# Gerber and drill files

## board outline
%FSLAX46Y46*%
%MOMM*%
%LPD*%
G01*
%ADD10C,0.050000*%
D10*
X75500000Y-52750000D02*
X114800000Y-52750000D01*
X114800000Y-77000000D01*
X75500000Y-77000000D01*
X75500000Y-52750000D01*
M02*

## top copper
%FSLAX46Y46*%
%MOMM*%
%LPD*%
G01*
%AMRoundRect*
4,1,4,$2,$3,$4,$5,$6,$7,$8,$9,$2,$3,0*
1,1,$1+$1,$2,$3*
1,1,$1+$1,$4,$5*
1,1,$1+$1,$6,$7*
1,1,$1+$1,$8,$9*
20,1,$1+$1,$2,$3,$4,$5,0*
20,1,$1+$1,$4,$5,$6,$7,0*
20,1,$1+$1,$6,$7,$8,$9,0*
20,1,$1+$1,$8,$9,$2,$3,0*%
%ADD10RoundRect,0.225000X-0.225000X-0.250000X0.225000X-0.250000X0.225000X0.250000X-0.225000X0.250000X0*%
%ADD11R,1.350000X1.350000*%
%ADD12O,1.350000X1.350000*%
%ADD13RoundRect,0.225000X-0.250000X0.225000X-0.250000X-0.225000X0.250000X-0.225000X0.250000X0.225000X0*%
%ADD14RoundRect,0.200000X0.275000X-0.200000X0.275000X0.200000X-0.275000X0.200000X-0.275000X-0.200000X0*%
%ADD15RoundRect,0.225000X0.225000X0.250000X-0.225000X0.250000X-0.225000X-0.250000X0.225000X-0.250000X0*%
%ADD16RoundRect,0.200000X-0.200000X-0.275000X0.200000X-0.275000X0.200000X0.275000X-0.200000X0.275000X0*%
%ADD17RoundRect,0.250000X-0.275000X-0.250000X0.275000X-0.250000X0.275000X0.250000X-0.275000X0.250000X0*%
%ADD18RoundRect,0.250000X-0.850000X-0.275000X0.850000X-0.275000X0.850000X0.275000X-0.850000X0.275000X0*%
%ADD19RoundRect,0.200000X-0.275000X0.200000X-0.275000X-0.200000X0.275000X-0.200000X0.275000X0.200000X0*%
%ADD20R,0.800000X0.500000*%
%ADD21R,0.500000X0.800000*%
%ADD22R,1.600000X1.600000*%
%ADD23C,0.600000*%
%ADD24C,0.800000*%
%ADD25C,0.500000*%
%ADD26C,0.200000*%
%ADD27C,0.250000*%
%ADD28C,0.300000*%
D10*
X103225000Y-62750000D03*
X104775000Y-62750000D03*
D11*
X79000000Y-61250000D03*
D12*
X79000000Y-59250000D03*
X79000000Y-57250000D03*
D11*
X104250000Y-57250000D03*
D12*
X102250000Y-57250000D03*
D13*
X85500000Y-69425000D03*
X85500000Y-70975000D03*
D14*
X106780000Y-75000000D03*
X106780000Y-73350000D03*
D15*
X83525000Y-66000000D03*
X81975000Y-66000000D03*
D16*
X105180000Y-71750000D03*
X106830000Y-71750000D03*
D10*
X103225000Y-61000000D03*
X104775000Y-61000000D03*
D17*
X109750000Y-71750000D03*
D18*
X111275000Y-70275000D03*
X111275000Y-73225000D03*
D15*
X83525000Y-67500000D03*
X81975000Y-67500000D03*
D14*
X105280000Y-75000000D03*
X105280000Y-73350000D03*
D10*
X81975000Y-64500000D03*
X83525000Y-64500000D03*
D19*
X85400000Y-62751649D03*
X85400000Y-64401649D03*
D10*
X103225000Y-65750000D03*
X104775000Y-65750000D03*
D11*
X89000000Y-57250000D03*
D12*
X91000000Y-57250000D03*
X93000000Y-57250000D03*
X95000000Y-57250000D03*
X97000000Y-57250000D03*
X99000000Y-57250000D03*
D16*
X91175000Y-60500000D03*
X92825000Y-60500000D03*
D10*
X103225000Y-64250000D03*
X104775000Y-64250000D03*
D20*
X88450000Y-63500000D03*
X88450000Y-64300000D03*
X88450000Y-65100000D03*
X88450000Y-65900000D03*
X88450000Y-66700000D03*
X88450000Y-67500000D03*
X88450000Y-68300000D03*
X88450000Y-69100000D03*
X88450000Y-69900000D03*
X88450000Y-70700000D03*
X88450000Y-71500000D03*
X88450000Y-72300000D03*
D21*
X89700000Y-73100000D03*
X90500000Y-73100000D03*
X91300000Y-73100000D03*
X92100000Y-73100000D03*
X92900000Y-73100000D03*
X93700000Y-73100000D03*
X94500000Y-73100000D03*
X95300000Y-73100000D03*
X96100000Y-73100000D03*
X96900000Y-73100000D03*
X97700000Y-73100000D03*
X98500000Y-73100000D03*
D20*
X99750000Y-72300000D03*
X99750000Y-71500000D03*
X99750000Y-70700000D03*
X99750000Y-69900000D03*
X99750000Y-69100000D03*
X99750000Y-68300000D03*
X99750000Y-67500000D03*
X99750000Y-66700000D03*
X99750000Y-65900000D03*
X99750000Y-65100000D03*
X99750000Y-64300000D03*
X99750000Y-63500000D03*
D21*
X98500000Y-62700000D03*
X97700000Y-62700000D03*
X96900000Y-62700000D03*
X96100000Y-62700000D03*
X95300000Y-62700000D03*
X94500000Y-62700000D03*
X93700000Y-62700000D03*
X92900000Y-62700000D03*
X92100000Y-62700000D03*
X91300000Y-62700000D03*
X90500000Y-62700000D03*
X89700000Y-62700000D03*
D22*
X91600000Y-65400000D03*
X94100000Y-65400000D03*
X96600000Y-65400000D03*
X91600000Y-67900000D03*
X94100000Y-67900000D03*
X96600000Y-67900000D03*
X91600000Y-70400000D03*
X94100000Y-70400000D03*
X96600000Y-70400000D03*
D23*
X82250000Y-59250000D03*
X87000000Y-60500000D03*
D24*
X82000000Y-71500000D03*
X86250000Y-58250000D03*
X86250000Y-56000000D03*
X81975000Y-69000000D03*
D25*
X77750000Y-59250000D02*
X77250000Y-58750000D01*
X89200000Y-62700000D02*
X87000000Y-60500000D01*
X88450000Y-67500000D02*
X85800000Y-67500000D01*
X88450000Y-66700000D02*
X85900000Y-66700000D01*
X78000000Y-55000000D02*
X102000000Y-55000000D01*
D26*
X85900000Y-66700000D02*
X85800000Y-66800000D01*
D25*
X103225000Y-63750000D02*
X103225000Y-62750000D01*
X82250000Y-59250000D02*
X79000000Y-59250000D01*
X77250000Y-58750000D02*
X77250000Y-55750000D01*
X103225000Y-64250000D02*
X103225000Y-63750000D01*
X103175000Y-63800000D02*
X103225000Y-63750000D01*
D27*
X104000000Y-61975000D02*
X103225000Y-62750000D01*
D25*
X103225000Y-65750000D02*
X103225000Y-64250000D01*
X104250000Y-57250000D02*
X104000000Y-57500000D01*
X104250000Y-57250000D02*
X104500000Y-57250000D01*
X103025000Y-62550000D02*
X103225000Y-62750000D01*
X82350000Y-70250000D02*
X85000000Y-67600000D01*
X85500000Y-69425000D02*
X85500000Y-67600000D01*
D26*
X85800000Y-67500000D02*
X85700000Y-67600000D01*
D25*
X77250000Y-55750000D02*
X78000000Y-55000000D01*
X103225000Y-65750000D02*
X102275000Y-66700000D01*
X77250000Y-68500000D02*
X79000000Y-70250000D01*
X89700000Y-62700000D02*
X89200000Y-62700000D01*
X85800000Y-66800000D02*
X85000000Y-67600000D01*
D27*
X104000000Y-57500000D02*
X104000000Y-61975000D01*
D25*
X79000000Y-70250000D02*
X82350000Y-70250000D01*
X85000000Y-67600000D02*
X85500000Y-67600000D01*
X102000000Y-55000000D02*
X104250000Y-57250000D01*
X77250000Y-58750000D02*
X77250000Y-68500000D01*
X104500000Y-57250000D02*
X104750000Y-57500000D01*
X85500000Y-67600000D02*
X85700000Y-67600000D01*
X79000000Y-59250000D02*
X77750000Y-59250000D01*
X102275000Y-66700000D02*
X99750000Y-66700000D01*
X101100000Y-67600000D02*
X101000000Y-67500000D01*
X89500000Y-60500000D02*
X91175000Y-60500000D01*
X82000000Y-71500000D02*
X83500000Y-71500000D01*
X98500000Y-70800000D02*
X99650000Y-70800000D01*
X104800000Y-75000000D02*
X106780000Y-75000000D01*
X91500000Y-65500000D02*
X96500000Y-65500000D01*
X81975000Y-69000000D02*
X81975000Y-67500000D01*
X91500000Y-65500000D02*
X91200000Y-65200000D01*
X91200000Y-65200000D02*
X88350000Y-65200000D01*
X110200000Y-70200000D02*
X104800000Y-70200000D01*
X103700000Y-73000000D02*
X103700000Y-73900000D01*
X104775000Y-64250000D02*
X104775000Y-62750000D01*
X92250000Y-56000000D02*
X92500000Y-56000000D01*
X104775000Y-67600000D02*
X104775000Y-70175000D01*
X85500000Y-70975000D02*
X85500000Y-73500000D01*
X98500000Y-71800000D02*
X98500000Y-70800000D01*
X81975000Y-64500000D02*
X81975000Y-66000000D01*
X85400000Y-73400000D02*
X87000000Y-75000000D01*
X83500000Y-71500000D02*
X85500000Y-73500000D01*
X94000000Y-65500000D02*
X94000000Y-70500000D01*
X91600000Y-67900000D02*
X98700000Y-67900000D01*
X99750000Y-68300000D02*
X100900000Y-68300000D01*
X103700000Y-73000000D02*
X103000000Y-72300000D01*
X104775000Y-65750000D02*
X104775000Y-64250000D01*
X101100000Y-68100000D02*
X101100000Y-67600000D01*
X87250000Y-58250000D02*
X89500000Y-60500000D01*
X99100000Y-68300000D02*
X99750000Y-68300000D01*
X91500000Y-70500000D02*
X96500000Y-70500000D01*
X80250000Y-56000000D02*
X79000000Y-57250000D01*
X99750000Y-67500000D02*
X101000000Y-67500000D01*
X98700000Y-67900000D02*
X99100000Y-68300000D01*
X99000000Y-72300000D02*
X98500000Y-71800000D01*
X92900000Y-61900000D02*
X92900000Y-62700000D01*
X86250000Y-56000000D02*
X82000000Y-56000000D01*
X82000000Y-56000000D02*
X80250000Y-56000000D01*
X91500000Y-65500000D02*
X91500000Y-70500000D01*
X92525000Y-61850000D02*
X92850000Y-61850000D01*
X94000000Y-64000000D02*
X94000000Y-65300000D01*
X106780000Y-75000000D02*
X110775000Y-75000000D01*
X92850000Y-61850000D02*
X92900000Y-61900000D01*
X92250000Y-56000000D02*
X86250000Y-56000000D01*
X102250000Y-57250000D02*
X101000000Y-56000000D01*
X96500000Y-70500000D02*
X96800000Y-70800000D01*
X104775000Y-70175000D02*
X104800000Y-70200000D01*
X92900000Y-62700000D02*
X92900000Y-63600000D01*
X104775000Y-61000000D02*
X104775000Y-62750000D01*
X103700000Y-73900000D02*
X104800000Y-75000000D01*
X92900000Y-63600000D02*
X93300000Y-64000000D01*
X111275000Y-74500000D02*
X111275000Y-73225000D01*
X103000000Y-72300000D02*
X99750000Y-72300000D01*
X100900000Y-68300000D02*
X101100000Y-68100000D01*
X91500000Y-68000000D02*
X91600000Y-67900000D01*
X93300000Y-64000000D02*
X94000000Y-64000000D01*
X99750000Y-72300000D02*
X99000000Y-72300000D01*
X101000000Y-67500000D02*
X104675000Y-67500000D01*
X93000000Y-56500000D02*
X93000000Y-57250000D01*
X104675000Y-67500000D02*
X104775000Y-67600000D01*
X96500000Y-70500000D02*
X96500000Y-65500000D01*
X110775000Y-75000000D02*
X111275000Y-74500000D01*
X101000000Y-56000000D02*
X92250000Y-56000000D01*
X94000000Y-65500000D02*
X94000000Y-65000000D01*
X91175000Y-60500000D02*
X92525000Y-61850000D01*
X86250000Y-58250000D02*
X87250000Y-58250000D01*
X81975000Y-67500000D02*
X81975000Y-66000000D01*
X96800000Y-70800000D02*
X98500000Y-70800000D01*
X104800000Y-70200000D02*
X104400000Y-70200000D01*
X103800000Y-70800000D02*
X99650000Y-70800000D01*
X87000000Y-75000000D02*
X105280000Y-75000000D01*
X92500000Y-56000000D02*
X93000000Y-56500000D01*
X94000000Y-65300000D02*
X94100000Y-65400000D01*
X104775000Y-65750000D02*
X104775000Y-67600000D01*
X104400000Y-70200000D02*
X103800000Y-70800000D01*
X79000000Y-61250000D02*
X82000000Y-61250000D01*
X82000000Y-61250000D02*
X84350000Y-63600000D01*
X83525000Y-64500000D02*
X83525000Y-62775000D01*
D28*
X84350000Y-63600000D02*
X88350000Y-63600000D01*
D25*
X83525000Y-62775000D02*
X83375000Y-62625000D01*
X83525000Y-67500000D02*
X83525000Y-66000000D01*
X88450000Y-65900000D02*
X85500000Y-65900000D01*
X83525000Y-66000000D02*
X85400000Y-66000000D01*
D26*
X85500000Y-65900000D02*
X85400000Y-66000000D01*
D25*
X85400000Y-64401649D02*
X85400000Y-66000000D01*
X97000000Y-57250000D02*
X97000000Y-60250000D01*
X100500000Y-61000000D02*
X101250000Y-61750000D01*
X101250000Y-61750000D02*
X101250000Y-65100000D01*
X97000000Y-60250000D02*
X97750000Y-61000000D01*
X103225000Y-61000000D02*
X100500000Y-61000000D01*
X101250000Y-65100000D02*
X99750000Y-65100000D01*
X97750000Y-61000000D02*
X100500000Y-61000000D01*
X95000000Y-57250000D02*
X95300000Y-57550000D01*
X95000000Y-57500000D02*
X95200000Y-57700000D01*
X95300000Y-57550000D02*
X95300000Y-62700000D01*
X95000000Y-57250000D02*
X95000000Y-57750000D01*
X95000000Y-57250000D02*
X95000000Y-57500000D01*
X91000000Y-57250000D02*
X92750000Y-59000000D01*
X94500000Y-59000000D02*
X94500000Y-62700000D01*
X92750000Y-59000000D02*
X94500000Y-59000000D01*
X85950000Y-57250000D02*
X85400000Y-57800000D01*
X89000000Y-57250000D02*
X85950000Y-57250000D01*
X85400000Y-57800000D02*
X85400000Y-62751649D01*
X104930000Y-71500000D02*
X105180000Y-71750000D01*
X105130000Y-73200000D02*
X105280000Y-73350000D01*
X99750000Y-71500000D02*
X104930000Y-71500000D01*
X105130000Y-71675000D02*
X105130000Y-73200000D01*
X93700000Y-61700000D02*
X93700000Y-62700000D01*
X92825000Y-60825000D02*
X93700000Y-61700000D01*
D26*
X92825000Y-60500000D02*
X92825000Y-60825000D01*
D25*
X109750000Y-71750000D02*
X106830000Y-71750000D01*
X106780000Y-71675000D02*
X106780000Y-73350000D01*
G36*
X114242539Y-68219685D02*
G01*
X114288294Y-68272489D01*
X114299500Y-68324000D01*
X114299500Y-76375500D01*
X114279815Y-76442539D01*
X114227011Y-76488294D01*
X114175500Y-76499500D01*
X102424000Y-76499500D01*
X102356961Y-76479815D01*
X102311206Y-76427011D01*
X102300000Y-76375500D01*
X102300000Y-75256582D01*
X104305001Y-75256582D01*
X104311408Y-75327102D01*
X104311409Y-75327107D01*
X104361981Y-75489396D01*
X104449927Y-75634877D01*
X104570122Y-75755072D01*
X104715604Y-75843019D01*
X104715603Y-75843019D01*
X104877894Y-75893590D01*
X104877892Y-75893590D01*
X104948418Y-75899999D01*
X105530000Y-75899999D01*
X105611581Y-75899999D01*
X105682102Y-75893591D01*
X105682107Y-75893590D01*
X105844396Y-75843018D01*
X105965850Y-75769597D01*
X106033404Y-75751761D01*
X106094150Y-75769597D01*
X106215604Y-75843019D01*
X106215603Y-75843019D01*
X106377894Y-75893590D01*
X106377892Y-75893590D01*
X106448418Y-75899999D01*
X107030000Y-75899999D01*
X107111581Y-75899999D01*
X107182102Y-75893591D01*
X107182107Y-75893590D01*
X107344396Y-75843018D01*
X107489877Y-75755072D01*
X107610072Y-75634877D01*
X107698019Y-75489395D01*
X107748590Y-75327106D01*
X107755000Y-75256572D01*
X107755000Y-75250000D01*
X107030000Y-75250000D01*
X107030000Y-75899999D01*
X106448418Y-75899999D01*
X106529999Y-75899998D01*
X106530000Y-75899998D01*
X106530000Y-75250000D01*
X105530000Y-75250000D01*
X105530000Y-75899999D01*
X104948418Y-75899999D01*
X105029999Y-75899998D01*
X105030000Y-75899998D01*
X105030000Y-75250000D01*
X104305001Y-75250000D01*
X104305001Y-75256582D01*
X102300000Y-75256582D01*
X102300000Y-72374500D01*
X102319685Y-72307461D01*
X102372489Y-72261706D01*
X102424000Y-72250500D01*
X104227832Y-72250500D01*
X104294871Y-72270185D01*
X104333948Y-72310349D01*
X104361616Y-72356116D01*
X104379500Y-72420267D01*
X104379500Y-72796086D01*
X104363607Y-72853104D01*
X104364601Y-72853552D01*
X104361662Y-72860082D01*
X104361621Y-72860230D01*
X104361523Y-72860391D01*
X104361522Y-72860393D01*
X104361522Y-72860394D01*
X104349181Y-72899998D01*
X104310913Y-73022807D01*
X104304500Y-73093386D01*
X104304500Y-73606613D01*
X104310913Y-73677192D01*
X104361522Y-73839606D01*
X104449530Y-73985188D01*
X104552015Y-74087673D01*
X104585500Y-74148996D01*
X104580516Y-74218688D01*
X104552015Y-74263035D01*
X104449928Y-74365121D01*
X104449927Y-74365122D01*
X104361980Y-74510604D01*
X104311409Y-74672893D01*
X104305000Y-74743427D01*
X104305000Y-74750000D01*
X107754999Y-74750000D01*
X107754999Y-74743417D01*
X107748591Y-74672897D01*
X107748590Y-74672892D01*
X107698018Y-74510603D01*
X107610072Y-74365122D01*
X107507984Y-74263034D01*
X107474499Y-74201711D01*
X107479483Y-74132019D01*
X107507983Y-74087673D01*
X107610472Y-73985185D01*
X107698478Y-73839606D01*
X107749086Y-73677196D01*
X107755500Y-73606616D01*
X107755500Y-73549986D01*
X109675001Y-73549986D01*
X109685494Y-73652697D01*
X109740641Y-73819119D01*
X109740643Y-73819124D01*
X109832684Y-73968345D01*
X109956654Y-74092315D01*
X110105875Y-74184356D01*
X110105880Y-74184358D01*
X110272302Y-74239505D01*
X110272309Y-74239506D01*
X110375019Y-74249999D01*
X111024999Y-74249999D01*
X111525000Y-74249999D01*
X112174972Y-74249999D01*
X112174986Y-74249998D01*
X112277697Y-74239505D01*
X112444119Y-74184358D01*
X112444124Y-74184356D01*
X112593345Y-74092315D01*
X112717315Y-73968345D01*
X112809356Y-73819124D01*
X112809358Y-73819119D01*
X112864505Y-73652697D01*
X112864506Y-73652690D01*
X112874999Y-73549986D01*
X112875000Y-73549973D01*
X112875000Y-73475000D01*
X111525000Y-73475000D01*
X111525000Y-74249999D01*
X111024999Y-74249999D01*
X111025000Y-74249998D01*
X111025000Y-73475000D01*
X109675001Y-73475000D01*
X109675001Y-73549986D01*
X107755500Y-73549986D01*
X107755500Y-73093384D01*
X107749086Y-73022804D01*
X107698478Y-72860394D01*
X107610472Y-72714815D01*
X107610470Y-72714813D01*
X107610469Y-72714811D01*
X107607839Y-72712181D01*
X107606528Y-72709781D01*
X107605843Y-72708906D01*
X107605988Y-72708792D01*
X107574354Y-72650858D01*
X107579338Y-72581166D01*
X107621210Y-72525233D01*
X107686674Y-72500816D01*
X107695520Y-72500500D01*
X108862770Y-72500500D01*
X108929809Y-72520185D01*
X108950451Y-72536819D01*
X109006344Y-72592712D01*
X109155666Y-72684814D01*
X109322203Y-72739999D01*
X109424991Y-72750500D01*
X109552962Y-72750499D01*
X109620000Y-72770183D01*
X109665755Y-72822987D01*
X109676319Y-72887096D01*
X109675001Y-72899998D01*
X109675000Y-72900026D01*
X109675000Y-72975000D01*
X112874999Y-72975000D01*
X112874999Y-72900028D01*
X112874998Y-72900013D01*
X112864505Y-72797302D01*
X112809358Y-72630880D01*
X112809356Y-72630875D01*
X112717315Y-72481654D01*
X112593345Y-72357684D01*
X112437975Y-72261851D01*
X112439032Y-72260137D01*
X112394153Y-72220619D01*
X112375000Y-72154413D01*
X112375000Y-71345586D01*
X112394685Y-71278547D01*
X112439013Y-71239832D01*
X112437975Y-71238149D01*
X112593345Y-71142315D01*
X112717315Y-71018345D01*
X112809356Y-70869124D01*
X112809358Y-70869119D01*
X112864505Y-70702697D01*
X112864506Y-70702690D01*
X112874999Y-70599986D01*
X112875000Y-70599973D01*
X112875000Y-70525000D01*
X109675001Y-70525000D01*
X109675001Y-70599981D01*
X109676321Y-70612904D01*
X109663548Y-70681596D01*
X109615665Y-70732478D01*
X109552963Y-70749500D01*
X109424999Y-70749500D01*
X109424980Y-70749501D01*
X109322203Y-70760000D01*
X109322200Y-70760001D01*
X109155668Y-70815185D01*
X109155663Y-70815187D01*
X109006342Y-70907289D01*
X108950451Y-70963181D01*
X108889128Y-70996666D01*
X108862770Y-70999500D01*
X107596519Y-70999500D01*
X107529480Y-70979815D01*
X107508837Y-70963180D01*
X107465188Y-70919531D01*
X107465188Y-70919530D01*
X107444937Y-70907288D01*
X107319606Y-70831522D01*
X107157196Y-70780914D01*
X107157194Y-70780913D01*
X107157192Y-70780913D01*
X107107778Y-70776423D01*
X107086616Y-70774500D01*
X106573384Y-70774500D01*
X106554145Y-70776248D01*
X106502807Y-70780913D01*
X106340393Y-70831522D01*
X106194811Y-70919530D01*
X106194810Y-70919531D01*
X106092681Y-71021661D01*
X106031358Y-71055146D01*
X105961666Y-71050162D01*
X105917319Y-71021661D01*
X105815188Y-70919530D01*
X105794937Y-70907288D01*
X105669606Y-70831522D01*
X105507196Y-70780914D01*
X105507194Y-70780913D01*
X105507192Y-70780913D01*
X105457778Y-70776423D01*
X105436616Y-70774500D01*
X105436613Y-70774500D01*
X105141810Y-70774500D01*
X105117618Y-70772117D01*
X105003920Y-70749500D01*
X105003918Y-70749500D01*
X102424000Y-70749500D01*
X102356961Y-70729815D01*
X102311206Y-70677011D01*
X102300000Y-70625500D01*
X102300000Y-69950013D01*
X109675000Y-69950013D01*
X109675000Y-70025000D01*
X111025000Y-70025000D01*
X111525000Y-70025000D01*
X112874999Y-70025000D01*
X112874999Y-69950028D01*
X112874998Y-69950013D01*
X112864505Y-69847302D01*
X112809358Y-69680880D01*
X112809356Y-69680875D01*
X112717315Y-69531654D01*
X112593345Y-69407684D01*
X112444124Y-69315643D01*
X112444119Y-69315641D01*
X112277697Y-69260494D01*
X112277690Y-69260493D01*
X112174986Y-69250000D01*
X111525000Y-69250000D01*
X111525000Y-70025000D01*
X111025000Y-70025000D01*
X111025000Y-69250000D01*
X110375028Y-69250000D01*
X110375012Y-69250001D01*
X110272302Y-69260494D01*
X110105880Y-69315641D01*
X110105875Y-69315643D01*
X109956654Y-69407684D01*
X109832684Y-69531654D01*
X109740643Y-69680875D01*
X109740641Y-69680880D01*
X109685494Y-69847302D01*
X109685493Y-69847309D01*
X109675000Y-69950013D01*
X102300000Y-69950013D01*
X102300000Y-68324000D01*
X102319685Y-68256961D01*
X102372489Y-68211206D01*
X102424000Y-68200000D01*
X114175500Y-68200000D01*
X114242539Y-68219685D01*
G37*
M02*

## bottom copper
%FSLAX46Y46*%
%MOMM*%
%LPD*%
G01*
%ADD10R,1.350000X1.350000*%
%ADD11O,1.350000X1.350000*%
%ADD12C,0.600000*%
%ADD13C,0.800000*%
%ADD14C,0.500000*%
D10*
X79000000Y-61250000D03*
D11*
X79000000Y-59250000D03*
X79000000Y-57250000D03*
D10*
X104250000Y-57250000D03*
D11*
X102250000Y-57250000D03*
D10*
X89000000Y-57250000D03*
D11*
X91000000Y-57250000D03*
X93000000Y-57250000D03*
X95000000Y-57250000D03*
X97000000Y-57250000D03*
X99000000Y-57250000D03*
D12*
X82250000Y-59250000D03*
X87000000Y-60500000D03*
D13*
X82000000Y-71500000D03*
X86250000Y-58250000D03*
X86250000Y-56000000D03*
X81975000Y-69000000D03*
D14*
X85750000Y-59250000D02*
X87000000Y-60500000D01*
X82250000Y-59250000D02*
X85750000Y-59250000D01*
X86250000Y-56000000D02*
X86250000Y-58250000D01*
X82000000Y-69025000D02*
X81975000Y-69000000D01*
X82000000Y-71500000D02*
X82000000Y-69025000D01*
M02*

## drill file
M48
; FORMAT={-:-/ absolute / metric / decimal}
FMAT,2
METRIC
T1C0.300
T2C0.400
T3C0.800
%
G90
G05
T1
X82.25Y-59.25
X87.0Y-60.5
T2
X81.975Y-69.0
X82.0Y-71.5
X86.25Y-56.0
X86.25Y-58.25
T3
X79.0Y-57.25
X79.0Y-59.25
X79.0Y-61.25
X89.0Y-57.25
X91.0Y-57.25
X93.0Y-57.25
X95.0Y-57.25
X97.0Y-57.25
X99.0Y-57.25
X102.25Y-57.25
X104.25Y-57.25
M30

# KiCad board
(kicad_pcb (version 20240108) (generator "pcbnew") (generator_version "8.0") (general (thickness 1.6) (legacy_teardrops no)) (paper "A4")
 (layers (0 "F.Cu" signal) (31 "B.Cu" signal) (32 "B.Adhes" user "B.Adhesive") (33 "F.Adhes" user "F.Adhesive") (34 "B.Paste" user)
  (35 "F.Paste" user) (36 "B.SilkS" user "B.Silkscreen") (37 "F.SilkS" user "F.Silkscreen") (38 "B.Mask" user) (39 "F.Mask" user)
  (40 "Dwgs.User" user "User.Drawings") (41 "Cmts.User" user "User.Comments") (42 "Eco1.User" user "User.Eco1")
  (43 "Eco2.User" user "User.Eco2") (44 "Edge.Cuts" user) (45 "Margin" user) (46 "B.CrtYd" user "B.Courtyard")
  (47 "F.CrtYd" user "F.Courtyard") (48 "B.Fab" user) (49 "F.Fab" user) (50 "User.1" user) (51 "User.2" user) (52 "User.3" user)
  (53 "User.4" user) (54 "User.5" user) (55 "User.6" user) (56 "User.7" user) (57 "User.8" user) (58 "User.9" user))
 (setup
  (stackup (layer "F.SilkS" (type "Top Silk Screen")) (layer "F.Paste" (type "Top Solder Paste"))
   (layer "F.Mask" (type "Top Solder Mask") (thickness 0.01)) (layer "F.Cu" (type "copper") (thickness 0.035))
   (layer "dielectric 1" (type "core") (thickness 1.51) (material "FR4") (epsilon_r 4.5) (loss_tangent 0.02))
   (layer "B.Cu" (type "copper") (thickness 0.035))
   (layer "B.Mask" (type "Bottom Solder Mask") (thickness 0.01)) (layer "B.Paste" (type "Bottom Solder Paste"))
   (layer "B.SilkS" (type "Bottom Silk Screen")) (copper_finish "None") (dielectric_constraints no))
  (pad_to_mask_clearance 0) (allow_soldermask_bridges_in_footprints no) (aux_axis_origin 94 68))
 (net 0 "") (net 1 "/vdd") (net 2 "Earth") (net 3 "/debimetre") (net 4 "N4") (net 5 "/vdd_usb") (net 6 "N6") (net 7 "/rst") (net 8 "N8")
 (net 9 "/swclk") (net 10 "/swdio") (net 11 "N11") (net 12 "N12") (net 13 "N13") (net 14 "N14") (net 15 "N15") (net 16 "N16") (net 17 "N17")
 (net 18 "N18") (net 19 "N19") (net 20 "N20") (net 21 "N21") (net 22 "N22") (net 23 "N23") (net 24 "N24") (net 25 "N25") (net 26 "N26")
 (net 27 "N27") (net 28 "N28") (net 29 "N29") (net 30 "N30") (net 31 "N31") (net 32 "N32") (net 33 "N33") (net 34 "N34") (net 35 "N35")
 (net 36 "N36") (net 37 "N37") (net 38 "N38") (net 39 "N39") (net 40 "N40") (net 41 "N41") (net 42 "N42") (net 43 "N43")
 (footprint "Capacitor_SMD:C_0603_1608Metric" (layer "F.Cu") (at 104 62.75)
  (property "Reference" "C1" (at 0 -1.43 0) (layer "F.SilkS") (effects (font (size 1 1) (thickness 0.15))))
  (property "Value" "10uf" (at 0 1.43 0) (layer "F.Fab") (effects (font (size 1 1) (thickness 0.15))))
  (pad "1" smd roundrect (at -0.775 0) (size 0.9 0.95) (layers "F.Cu" "F.Paste" "F.Mask") (roundrect_rratio 0.25) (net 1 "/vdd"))
  (pad "2" smd roundrect (at 0.775 0) (size 0.9 0.95) (layers "F.Cu" "F.Paste" "F.Mask") (roundrect_rratio 0.25) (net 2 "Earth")))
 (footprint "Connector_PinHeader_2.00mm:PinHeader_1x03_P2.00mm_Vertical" (layer "F.Cu") (at 79 61.25 180)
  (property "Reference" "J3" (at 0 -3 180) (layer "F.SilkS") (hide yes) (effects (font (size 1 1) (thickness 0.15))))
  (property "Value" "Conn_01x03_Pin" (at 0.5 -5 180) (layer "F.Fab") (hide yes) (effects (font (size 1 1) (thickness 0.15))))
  (pad "1" thru_hole rect (at 0 0 180) (size 1.35 1.35) (drill 0.8) (layers "*.Cu" "*.Mask") (remove_unused_layers no) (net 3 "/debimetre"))
  (pad "2" thru_hole oval (at 0 2 180) (size 1.35 1.35) (drill 0.8) (layers "*.Cu" "*.Mask") (remove_unused_layers no) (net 1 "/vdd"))
  (pad "3" thru_hole oval (at 0 4 180) (size 1.35 1.35) (drill 0.8) (layers "*.Cu" "*.Mask") (remove_unused_layers no) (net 2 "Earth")))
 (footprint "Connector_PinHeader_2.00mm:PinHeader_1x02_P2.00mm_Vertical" (layer "F.Cu") (at 104.25 57.25 -90)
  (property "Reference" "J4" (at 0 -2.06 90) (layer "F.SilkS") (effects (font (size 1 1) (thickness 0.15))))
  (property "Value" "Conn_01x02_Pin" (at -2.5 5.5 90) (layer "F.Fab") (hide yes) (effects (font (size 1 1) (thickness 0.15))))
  (pad "1" thru_hole rect (at 0 0 270) (size 1.35 1.35) (drill 0.8) (layers "*.Cu" "*.Mask") (remove_unused_layers no) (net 1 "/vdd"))
  (pad "2" thru_hole oval (at 0 2 270) (size 1.35 1.35) (drill 0.8) (layers "*.Cu" "*.Mask") (remove_unused_layers no) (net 2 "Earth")))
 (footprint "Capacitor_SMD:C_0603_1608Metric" (layer "F.Cu") (at 85.5 70.2 -90)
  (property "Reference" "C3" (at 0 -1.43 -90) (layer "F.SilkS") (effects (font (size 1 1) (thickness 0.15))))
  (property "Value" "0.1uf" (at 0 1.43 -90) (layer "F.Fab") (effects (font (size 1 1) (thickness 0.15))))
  (pad "1" smd roundrect (at -0.775 0 270) (size 0.9 0.95) (layers "F.Cu" "F.Paste" "F.Mask") (roundrect_rratio 0.25) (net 1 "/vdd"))
  (pad "2" smd roundrect (at 0.775 0 270) (size 0.9 0.95) (layers "F.Cu" "F.Paste" "F.Mask") (roundrect_rratio 0.25) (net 2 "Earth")))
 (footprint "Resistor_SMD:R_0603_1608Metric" (layer "F.Cu") (at 106.78 74.175 90)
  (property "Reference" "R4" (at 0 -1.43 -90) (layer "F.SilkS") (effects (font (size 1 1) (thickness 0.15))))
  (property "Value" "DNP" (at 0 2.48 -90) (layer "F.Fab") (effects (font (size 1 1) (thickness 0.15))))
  (pad "1" smd roundrect (at -0.825 0 90) (size 0.8 0.95) (layers "F.Cu" "F.Paste" "F.Mask") (roundrect_rratio 0.25) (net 2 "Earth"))
  (pad "2" smd roundrect (at 0.825 0 90) (size 0.8 0.95) (layers "F.Cu" "F.Paste" "F.Mask") (roundrect_rratio 0.25) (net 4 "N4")))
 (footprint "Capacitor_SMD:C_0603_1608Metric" (layer "F.Cu") (at 82.75 66 180)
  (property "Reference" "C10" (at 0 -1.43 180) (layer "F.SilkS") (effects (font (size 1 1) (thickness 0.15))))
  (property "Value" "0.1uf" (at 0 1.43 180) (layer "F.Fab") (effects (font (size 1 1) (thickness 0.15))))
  (pad "1" smd roundrect (at -0.775 0 180) (size 0.9 0.95) (layers "F.Cu" "F.Paste" "F.Mask") (roundrect_rratio 0.25) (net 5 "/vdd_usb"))
  (pad "2" smd roundrect (at 0.775 0 180) (size 0.9 0.95) (layers "F.Cu" "F.Paste" "F.Mask") (roundrect_rratio 0.25) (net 2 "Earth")))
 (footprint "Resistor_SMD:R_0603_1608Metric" (layer "F.Cu") (at 106.005 71.75)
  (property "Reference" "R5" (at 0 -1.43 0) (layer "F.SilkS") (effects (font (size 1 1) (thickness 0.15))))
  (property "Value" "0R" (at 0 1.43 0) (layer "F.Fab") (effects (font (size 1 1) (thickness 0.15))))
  (pad "1" smd roundrect (at -0.825 0) (size 0.8 0.95) (layers "F.Cu" "F.Paste" "F.Mask") (roundrect_rratio 0.25) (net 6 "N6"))
  (pad "2" smd roundrect (at 0.825 0) (size 0.8 0.95) (layers "F.Cu" "F.Paste" "F.Mask") (roundrect_rratio 0.25) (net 4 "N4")))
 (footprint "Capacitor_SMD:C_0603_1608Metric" (layer "F.Cu") (at 104 61)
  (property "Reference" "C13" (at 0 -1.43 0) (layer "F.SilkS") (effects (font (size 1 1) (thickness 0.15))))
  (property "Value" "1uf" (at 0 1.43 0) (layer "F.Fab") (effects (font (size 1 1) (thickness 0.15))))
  (pad "1" smd roundrect (at -0.775 0) (size 0.9 0.95) (layers "F.Cu" "F.Paste" "F.Mask") (roundrect_rratio 0.25) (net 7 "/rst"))
  (pad "2" smd roundrect (at 0.775 0) (size 0.9 0.95) (layers "F.Cu" "F.Paste" "F.Mask") (roundrect_rratio 0.25) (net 2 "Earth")))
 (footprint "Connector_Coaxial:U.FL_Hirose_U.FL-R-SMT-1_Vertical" (layer "F.Cu") (at 110.8 71.75)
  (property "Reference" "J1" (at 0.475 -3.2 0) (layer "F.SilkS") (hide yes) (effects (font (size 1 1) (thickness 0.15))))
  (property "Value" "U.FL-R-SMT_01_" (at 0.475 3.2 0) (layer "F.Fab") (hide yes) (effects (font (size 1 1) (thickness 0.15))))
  (pad "1" smd roundrect (at -1.05 0) (size 1.05 1) (layers "F.Cu" "F.Paste" "F.Mask") (roundrect_rratio 0.25) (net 4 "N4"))
  (pad "2" smd roundrect (at 0.475 -1.475) (size 2.2 1.05) (layers "F.Cu" "F.Paste" "F.Mask") (roundrect_rratio 0.2380952381)
   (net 2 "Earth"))
  (pad "2" smd roundrect (at 0.475 1.475) (size 2.2 1.05) (layers "F.Cu" "F.Paste" "F.Mask") (roundrect_rratio 0.2380952381) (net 2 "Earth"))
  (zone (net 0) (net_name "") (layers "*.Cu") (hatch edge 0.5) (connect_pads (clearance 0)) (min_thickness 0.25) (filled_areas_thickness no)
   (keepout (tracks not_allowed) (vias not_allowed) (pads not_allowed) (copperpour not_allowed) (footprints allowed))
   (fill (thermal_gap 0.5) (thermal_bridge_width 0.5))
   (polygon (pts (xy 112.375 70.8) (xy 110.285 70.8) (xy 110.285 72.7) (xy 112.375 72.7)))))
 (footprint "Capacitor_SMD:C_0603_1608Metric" (layer "F.Cu") (at 82.75 67.5 180)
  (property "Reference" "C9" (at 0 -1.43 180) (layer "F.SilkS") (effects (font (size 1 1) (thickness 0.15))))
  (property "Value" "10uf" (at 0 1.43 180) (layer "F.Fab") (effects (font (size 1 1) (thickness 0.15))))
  (pad "1" smd roundrect (at -0.775 0 180) (size 0.9 0.95) (layers "F.Cu" "F.Paste" "F.Mask") (roundrect_rratio 0.25) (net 5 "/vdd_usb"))
  (pad "2" smd roundrect (at 0.775 0 180) (size 0.9 0.95) (layers "F.Cu" "F.Paste" "F.Mask") (roundrect_rratio 0.25) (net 2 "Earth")))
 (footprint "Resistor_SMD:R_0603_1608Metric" (layer "F.Cu") (at 105.28 74.175 90)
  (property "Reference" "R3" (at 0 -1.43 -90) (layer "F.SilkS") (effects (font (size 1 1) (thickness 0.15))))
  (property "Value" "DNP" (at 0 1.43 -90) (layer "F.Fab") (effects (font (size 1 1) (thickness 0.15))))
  (pad "1" smd roundrect (at -0.825 0 90) (size 0.8 0.95) (layers "F.Cu" "F.Paste" "F.Mask") (roundrect_rratio 0.25) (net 2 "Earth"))
  (pad "2" smd roundrect (at 0.825 0 90) (size 0.8 0.95) (layers "F.Cu" "F.Paste" "F.Mask") (roundrect_rratio 0.25) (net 6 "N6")))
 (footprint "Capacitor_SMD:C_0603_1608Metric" (layer "F.Cu") (at 82.75 64.5)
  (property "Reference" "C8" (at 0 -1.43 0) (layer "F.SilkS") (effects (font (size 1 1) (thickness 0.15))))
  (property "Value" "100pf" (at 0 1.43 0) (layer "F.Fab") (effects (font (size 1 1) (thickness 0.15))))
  (pad "1" smd roundrect (at -0.775 0) (size 0.9 0.95) (layers "F.Cu" "F.Paste" "F.Mask") (roundrect_rratio 0.25) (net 2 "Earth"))
  (pad "2" smd roundrect (at 0.775 0) (size 0.9 0.95) (layers "F.Cu" "F.Paste" "F.Mask") (roundrect_rratio 0.25) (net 3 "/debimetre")))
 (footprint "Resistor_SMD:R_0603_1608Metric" (layer "F.Cu") (at 85.4 63.576649 -90)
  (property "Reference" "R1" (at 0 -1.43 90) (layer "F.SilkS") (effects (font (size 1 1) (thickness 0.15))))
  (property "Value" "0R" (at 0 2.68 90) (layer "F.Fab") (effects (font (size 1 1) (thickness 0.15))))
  (pad "1" smd roundrect (at -0.825 0 270) (size 0.8 0.95) (layers "F.Cu" "F.Paste" "F.Mask") (roundrect_rratio 0.25) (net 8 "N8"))
  (pad "2" smd roundrect (at 0.825 0 270) (size 0.8 0.95) (layers "F.Cu" "F.Paste" "F.Mask") (roundrect_rratio 0.25) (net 5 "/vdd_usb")))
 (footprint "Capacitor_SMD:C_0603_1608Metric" (layer "F.Cu") (at 104 65.75)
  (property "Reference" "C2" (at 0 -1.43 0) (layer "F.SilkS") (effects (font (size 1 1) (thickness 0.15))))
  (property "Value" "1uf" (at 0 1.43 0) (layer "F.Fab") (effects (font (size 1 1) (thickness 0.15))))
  (pad "1" smd roundrect (at -0.775 0) (size 0.9 0.95) (layers "F.Cu" "F.Paste" "F.Mask") (roundrect_rratio 0.25) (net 1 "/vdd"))
  (pad "2" smd roundrect (at 0.775 0) (size 0.9 0.95) (layers "F.Cu" "F.Paste" "F.Mask") (roundrect_rratio 0.25) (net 2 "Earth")))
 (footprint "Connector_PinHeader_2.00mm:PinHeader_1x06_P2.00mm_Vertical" (layer "F.Cu") (at 89 57.25 90)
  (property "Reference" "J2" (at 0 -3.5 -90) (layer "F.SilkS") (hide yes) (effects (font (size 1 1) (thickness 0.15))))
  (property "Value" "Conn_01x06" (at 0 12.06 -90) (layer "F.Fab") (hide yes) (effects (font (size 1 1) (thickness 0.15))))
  (pad "1" thru_hole rect (at 0 0 90) (size 1.35 1.35) (drill 0.8) (layers "*.Cu" "*.Mask") (remove_unused_layers no) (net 8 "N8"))
  (pad "2" thru_hole oval (at 0 2 90) (size 1.35 1.35) (drill 0.8) (layers "*.Cu" "*.Mask") (remove_unused_layers no) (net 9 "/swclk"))
  (pad "3" thru_hole oval (at 0 4 90) (size 1.35 1.35) (drill 0.8) (layers "*.Cu" "*.Mask") (remove_unused_layers no) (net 2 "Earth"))
  (pad "4" thru_hole oval (at 0 6 90) (size 1.35 1.35) (drill 0.8) (layers "*.Cu" "*.Mask") (remove_unused_layers no) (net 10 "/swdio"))
  (pad "5" thru_hole oval (at 0 8 90) (size 1.35 1.35) (drill 0.8) (layers "*.Cu" "*.Mask") (remove_unused_layers no) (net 7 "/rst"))
  (pad "6" thru_hole oval (at 0 10 90) (size 1.35 1.35) (drill 0.8) (layers "*.Cu" "*.Mask") (remove_unused_layers no) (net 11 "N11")))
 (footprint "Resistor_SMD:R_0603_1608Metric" (layer "F.Cu") (at 92 60.5)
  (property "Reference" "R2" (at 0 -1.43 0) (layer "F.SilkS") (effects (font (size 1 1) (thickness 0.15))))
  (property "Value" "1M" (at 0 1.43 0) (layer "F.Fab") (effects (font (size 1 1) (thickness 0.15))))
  (pad "1" smd roundrect (at -0.825 0) (size 0.8 0.95) (layers "F.Cu" "F.Paste" "F.Mask") (roundrect_rratio 0.25) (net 2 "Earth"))
  (pad "2" smd roundrect (at 0.825 0) (size 0.8 0.95) (layers "F.Cu" "F.Paste" "F.Mask") (roundrect_rratio 0.25) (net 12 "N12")))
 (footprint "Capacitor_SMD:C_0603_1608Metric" (layer "F.Cu") (at 104 64.25)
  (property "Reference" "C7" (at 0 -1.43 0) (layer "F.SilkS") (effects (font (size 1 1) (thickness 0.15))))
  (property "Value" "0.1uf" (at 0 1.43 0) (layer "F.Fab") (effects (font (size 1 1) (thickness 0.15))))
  (pad "1" smd roundrect (at -0.775 0) (size 0.9 0.95) (layers "F.Cu" "F.Paste" "F.Mask") (roundrect_rratio 0.25) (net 1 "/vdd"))
  (pad "2" smd roundrect (at 0.775 0) (size 0.9 0.95) (layers "F.Cu" "F.Paste" "F.Mask") (roundrect_rratio 0.25) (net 2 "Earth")))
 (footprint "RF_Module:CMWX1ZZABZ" (layer "F.Cu") (at 94.1 67.9)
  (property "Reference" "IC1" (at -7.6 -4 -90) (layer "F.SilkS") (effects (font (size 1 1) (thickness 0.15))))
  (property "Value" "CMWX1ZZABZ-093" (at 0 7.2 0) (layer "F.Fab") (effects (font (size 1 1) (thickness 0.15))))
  (pad "1" smd rect (at -5.65 -4.4) (size 0.8 0.5) (layers "F.Cu" "F.Paste" "F.Mask") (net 3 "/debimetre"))
  (pad "2" smd rect (at -5.65 -3.6) (size 0.8 0.5) (layers "F.Cu" "F.Paste" "F.Mask") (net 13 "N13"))
  (pad "3" smd rect (at -5.65 -2.8) (size 0.8 0.5) (layers "F.Cu" "F.Paste" "F.Mask") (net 2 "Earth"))
  (pad "4" smd rect (at -5.65 -2) (size 0.8 0.5) (layers "F.Cu" "F.Paste" "F.Mask") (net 5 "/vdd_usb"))
  (pad "5" smd rect (at -5.65 -1.2) (size 0.8 0.5) (layers "F.Cu" "F.Paste" "F.Mask") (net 1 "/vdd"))
  (pad "6" smd rect (at -5.65 -0.4) (size 0.8 0.5) (layers "F.Cu" "F.Paste" "F.Mask") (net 1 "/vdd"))
  (pad "7" smd rect (at -5.65 0.4) (size 0.8 0.5) (layers "F.Cu" "F.Paste" "F.Mask") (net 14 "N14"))
  (pad "8" smd rect (at -5.65 1.2) (size 0.8 0.5) (layers "F.Cu" "F.Paste" "F.Mask") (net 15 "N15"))
  (pad "9" smd rect (at -5.65 2) (size 0.8 0.5) (layers "F.Cu" "F.Paste" "F.Mask") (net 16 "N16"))
  (pad "10" smd rect (at -5.65 2.8) (size 0.8 0.5) (layers "F.Cu" "F.Paste" "F.Mask") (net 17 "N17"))
  (pad "11" smd rect (at -5.65 3.6) (size 0.8 0.5) (layers "F.Cu" "F.Paste" "F.Mask") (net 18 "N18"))
  (pad "12" smd rect (at -5.65 4.4) (size 0.8 0.5) (layers "F.Cu" "F.Paste" "F.Mask") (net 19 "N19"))
  (pad "13" smd rect (at -4.4 5.2 90) (size 0.8 0.5) (layers "F.Cu" "F.Paste" "F.Mask") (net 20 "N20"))
  (pad "14" smd rect (at -3.6 5.2 90) (size 0.8 0.5) (layers "F.Cu" "F.Paste" "F.Mask") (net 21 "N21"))
  (pad "15" smd rect (at -2.8 5.2 90) (size 0.8 0.5) (layers "F.Cu" "F.Paste" "F.Mask") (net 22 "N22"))
  (pad "16" smd rect (at -2 5.2 90) (size 0.8 0.5) (layers "F.Cu" "F.Paste" "F.Mask") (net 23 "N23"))
  (pad "17" smd rect (at -1.2 5.2 90) (size 0.8 0.5) (layers "F.Cu" "F.Paste" "F.Mask") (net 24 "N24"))
  (pad "18" smd rect (at -0.4 5.2 90) (size 0.8 0.5) (layers "F.Cu" "F.Paste" "F.Mask") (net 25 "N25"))
  (pad "19" smd rect (at 0.4 5.2 90) (size 0.8 0.5) (layers "F.Cu" "F.Paste" "F.Mask") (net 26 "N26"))
  (pad "20" smd rect (at 1.2 5.2 270) (size 0.8 0.5) (layers "F.Cu" "F.Paste" "F.Mask") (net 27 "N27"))
  (pad "21" smd rect (at 2 5.2 270) (size 0.8 0.5) (layers "F.Cu" "F.Paste" "F.Mask") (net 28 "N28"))
  (pad "22" smd rect (at 2.8 5.2 270) (size 0.8 0.5) (layers "F.Cu" "F.Paste" "F.Mask") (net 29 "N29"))
  (pad "23" smd rect (at 3.6 5.2 270) (size 0.8 0.5) (layers "F.Cu" "F.Paste" "F.Mask") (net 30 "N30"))
  (pad "24" smd rect (at 4.4 5.2 270) (size 0.8 0.5) (layers "F.Cu" "F.Paste" "F.Mask") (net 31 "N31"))
  (pad "25" smd rect (at 5.65 4.4) (size 0.8 0.5) (layers "F.Cu" "F.Paste" "F.Mask") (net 2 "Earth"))
  (pad "26" smd rect (at 5.65 3.6) (size 0.8 0.5) (layers "F.Cu" "F.Paste" "F.Mask") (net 6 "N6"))
  (pad "27" smd rect (at 5.65 2.8) (size 0.8 0.5) (layers "F.Cu" "F.Paste" "F.Mask") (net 2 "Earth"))
  (pad "28" smd rect (at 5.65 2) (size 0.8 0.5) (layers "F.Cu" "F.Paste" "F.Mask") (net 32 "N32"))
  (pad "29" smd rect (at 5.65 1.2) (size 0.8 0.5) (layers "F.Cu" "F.Paste" "F.Mask") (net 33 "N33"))
  (pad "30" smd rect (at 5.65 0.4) (size 0.8 0.5) (layers "F.Cu" "F.Paste" "F.Mask") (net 2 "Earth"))
  (pad "31" smd rect (at 5.65 -0.4) (size 0.8 0.5) (layers "F.Cu" "F.Paste" "F.Mask") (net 2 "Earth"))
  (pad "32" smd rect (at 5.65 -1.2) (size 0.8 0.5) (layers "F.Cu" "F.Paste" "F.Mask") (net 1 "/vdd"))
  (pad "33" smd rect (at 5.65 -2) (size 0.8 0.5) (layers "F.Cu" "F.Paste" "F.Mask") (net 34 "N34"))
  (pad "34" smd rect (at 5.65 -2.8) (size 0.8 0.5) (layers "F.Cu" "F.Paste" "F.Mask") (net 7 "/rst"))
  (pad "35" smd rect (at 5.65 -3.6) (size 0.8 0.5) (layers "F.Cu" "F.Paste" "F.Mask") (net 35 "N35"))
  (pad "36" smd rect (at 5.65 -4.4) (size 0.8 0.5) (layers "F.Cu" "F.Paste" "F.Mask") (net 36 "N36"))
  (pad "37" smd rect (at 4.4 -5.2 90) (size 0.8 0.5) (layers "F.Cu" "F.Paste" "F.Mask") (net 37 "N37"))
  (pad "38" smd rect (at 3.6 -5.2 90) (size 0.8 0.5) (layers "F.Cu" "F.Paste" "F.Mask") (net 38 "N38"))
  (pad "39" smd rect (at 2.8 -5.2 90) (size 0.8 0.5) (layers "F.Cu" "F.Paste" "F.Mask") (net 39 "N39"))
  (pad "40" smd rect (at 2 -5.2 90) (size 0.8 0.5) (layers "F.Cu" "F.Paste" "F.Mask") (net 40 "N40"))
  (pad "41" smd rect (at 1.2 -5.2 90) (size 0.8 0.5) (layers "F.Cu" "F.Paste" "F.Mask") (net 10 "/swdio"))
  (pad "42" smd rect (at 0.4 -5.2 90) (size 0.8 0.5) (layers "F.Cu" "F.Paste" "F.Mask") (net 9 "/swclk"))
  (pad "43" smd rect (at -0.4 -5.2 90) (size 0.8 0.5) (layers "F.Cu" "F.Paste" "F.Mask") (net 12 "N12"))
  (pad "44" smd rect (at -1.2 -5.2 90) (size 0.8 0.5) (layers "F.Cu" "F.Paste" "F.Mask") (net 2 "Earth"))
  (pad "45" smd rect (at -2 -5.2 90) (size 0.8 0.5) (layers "F.Cu" "F.Paste" "F.Mask") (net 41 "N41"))
  (pad "46" smd rect (at -2.8 -5.2 90) (size 0.8 0.5) (layers "F.Cu" "F.Paste" "F.Mask") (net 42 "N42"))
  (pad "47" smd rect (at -3.6 -5.2 90) (size 0.8 0.5) (layers "F.Cu" "F.Paste" "F.Mask") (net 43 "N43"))
  (pad "48" smd rect (at -4.4 -5.2 90) (size 0.8 0.5) (layers "F.Cu" "F.Paste" "F.Mask") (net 1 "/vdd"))
  (pad "49" smd rect (at -2.5 -2.5 90) (size 1.6 1.6) (layers "F.Cu" "F.Paste" "F.Mask") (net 2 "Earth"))
  (pad "50" smd rect (at 0 -2.5 90) (size 1.6 1.6) (layers "F.Cu" "F.Paste" "F.Mask") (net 2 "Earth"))
  (pad "51" smd rect (at 2.5 -2.5 90) (size 1.6 1.6) (layers "F.Cu" "F.Paste" "F.Mask") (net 2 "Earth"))
  (pad "52" smd rect (at -2.5 0 90) (size 1.6 1.6) (layers "F.Cu" "F.Paste" "F.Mask") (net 2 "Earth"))
  (pad "53" smd rect (at 0 0 90) (size 1.6 1.6) (layers "F.Cu" "F.Paste" "F.Mask") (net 2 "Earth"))
  (pad "54" smd rect (at 2.5 0 90) (size 1.6 1.6) (layers "F.Cu" "F.Paste" "F.Mask") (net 2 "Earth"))
  (pad "55" smd rect (at -2.5 2.5 90) (size 1.6 1.6) (layers "F.Cu" "F.Paste" "F.Mask") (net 2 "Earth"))
  (pad "56" smd rect (at 0 2.5 90) (size 1.6 1.6) (layers "F.Cu" "F.Paste" "F.Mask") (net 2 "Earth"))
  (pad "57" smd rect (at 2.5 2.5 90) (size 1.6 1.6) (layers "F.Cu" "F.Paste" "F.Mask") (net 2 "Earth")))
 (gr_rect (start 75.5 52.75) (end 114.8 77) (stroke (width 0.05) (type default)) (fill none) (layer "Edge.Cuts"))
 (segment (start 77.75 59.25) (end 77.25 58.75) (width 0.5) (layer "F.Cu") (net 1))
 (segment (start 89.2 62.7) (end 87 60.5) (width 0.5) (layer "F.Cu") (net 1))
 (segment (start 88.45 67.5) (end 85.8 67.5) (width 0.5) (layer "F.Cu") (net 1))
 (segment (start 88.45 66.7) (end 85.9 66.7) (width 0.5) (layer "F.Cu") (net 1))
 (segment (start 78 55) (end 102 55) (width 0.5) (layer "F.Cu") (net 1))
 (segment (start 85.9 66.7) (end 85.8 66.8) (width 0.2) (layer "F.Cu") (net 1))
 (segment (start 103.225 63.75) (end 103.225 62.75) (width 0.5) (layer "F.Cu") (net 1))
 (segment (start 82.25 59.25) (end 79 59.25) (width 0.5) (layer "F.Cu") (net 1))
 (segment (start 77.25 58.75) (end 77.25 55.75) (width 0.5) (layer "F.Cu") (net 1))
 (segment (start 103.225 64.25) (end 103.225 63.75) (width 0.5) (layer "F.Cu") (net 1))
 (segment (start 103.175 63.8) (end 103.225 63.75) (width 0.5) (layer "F.Cu") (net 1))
 (segment (start 104 61.975) (end 103.225 62.75) (width 0.25) (layer "F.Cu") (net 1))
 (segment (start 103.225 65.75) (end 103.225 64.25) (width 0.5) (layer "F.Cu") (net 1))
 (segment (start 104.25 57.25) (end 104 57.5) (width 0.5) (layer "F.Cu") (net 1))
 (segment (start 104.25 57.25) (end 104.5 57.25) (width 0.5) (layer "F.Cu") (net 1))
 (segment (start 103.025 62.55) (end 103.225 62.75) (width 0.5) (layer "F.Cu") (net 1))
 (segment (start 82.35 70.25) (end 85 67.6) (width 0.5) (layer "F.Cu") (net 1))
 (segment (start 85.5 69.425) (end 85.5 67.6) (width 0.5) (layer "F.Cu") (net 1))
 (segment (start 85.8 67.5) (end 85.7 67.6) (width 0.2) (layer "F.Cu") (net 1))
 (segment (start 77.25 55.75) (end 78 55) (width 0.5) (layer "F.Cu") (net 1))
 (segment (start 103.225 65.75) (end 102.275 66.7) (width 0.5) (layer "F.Cu") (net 1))
 (segment (start 77.25 68.5) (end 79 70.25) (width 0.5) (layer "F.Cu") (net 1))
 (segment (start 89.7 62.7) (end 89.2 62.7) (width 0.5) (layer "F.Cu") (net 1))
 (segment (start 85.8 66.8) (end 85 67.6) (width 0.5) (layer "F.Cu") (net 1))
 (segment (start 104 57.5) (end 104 61.975) (width 0.25) (layer "F.Cu") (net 1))
 (segment (start 79 70.25) (end 82.35 70.25) (width 0.5) (layer "F.Cu") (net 1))
 (segment (start 85 67.6) (end 85.5 67.6) (width 0.5) (layer "F.Cu") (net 1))
 (segment (start 102 55) (end 104.25 57.25) (width 0.5) (layer "F.Cu") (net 1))
 (segment (start 77.25 58.75) (end 77.25 68.5) (width 0.5) (layer "F.Cu") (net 1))
 (segment (start 104.5 57.25) (end 104.75 57.5) (width 0.5) (layer "F.Cu") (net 1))
 (segment (start 85.5 67.6) (end 85.7 67.6) (width 0.5) (layer "F.Cu") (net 1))
 (segment (start 79 59.25) (end 77.75 59.25) (width 0.5) (layer "F.Cu") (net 1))
 (segment (start 102.275 66.7) (end 99.75 66.7) (width 0.5) (layer "F.Cu") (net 1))
 (via (at 82.25 59.25) (size 0.6) (drill 0.3) (layers "F.Cu" "B.Cu") (free yes) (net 1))
 (via (at 87 60.5) (size 0.6) (drill 0.3) (layers "F.Cu" "B.Cu") (free yes) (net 1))
 (segment (start 85.75 59.25) (end 87 60.5) (width 0.5) (layer "B.Cu") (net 1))
 (segment (start 82.25 59.25) (end 85.75 59.25) (width 0.5) (layer "B.Cu") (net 1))
 (segment (start 101.1 67.6) (end 101 67.5) (width 0.5) (layer "F.Cu") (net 2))
 (segment (start 89.5 60.5) (end 91.175 60.5) (width 0.5) (layer "F.Cu") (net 2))
 (segment (start 82 71.5) (end 83.5 71.5) (width 0.5) (layer "F.Cu") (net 2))
 (segment (start 98.5 70.8) (end 99.65 70.8) (width 0.5) (layer "F.Cu") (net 2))
 (segment (start 104.8 75) (end 106.78 75) (width 0.5) (layer "F.Cu") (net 2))
 (segment (start 91.5 65.5) (end 96.5 65.5) (width 0.5) (layer "F.Cu") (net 2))
 (segment (start 81.975 69) (end 81.975 67.5) (width 0.5) (layer "F.Cu") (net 2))
 (segment (start 91.5 65.5) (end 91.2 65.2) (width 0.5) (layer "F.Cu") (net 2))
 (segment (start 91.2 65.2) (end 88.35 65.2) (width 0.5) (layer "F.Cu") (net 2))
 (segment (start 110.2 70.2) (end 104.8 70.2) (width 0.5) (layer "F.Cu") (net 2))
 (segment (start 103.7 73) (end 103.7 73.9) (width 0.5) (layer "F.Cu") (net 2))
 (segment (start 104.775 64.25) (end 104.775 62.75) (width 0.5) (layer "F.Cu") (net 2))
 (segment (start 92.25 56) (end 92.5 56) (width 0.5) (layer "F.Cu") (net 2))
 (segment (start 104.775 67.6) (end 104.775 70.175) (width 0.5) (layer "F.Cu") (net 2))
 (segment (start 85.5 70.975) (end 85.5 73.5) (width 0.5) (layer "F.Cu") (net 2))
 (segment (start 98.5 71.8) (end 98.5 70.8) (width 0.5) (layer "F.Cu") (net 2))
 (segment (start 81.975 64.5) (end 81.975 66) (width 0.5) (layer "F.Cu") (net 2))
 (segment (start 85.4 73.4) (end 87 75) (width 0.5) (layer "F.Cu") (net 2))
 (segment (start 83.5 71.5) (end 85.5 73.5) (width 0.5) (layer "F.Cu") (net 2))
 (segment (start 94 65.5) (end 94 70.5) (width 0.5) (layer "F.Cu") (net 2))
 (segment (start 91.6 67.9) (end 98.7 67.9) (width 0.5) (layer "F.Cu") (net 2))
 (segment (start 99.75 68.3) (end 100.9 68.3) (width 0.5) (layer "F.Cu") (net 2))
 (segment (start 103.7 73) (end 103 72.3) (width 0.5) (layer "F.Cu") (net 2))
 (segment (start 104.775 65.75) (end 104.775 64.25) (width 0.5) (layer "F.Cu") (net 2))
 (segment (start 101.1 68.1) (end 101.1 67.6) (width 0.5) (layer "F.Cu") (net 2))
 (segment (start 87.25 58.25) (end 89.5 60.5) (width 0.5) (layer "F.Cu") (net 2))
 (segment (start 99.1 68.3) (end 99.75 68.3) (width 0.5) (layer "F.Cu") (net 2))
 (segment (start 91.5 70.5) (end 96.5 70.5) (width 0.5) (layer "F.Cu") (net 2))
 (segment (start 80.25 56) (end 79 57.25) (width 0.5) (layer "F.Cu") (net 2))
 (segment (start 99.75 67.5) (end 101 67.5) (width 0.5) (layer "F.Cu") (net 2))
 (segment (start 98.7 67.9) (end 99.1 68.3) (width 0.5) (layer "F.Cu") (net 2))
 (segment (start 99 72.3) (end 98.5 71.8) (width 0.5) (layer "F.Cu") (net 2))
 (segment (start 92.9 61.9) (end 92.9 62.7) (width 0.5) (layer "F.Cu") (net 2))
 (segment (start 86.25 56) (end 82 56) (width 0.5) (layer "F.Cu") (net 2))
 (segment (start 82 56) (end 80.25 56) (width 0.5) (layer "F.Cu") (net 2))
 (segment (start 91.5 65.5) (end 91.5 70.5) (width 0.5) (layer "F.Cu") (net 2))
 (segment (start 92.525 61.85) (end 92.85 61.85) (width 0.5) (layer "F.Cu") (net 2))
 (segment (start 94 64) (end 94 65.3) (width 0.5) (layer "F.Cu") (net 2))
 (segment (start 106.78 75) (end 110.775 75) (width 0.5) (layer "F.Cu") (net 2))
 (segment (start 92.85 61.85) (end 92.9 61.9) (width 0.5) (layer "F.Cu") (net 2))
 (segment (start 92.25 56) (end 86.25 56) (width 0.5) (layer "F.Cu") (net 2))
 (segment (start 102.25 57.25) (end 101 56) (width 0.5) (layer "F.Cu") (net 2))
 (segment (start 96.5 70.5) (end 96.8 70.8) (width 0.5) (layer "F.Cu") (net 2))
 (segment (start 104.775 70.175) (end 104.8 70.2) (width 0.5) (layer "F.Cu") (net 2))
 (segment (start 92.9 62.7) (end 92.9 63.6) (width 0.5) (layer "F.Cu") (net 2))
 (segment (start 104.775 61) (end 104.775 62.75) (width 0.5) (layer "F.Cu") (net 2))
 (segment (start 103.7 73.9) (end 104.8 75) (width 0.5) (layer "F.Cu") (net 2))
 (segment (start 92.9 63.6) (end 93.3 64) (width 0.5) (layer "F.Cu") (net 2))
 (segment (start 111.275 74.5) (end 111.275 73.225) (width 0.5) (layer "F.Cu") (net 2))
 (segment (start 103 72.3) (end 99.75 72.3) (width 0.5) (layer "F.Cu") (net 2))
 (segment (start 100.9 68.3) (end 101.1 68.1) (width 0.5) (layer "F.Cu") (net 2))
 (segment (start 91.5 68) (end 91.6 67.9) (width 0.5) (layer "F.Cu") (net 2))
 (segment (start 93.3 64) (end 94 64) (width 0.5) (layer "F.Cu") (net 2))
 (segment (start 99.75 72.3) (end 99 72.3) (width 0.5) (layer "F.Cu") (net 2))
 (segment (start 101 67.5) (end 104.675 67.5) (width 0.5) (layer "F.Cu") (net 2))
 (segment (start 93 56.5) (end 93 57.25) (width 0.5) (layer "F.Cu") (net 2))
 (segment (start 104.675 67.5) (end 104.775 67.6) (width 0.5) (layer "F.Cu") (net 2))
 (segment (start 96.5 70.5) (end 96.5 65.5) (width 0.5) (layer "F.Cu") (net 2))
 (segment (start 110.775 75) (end 111.275 74.5) (width 0.5) (layer "F.Cu") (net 2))
 (segment (start 101 56) (end 92.25 56) (width 0.5) (layer "F.Cu") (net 2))
 (segment (start 94 65.5) (end 94 65) (width 0.5) (layer "F.Cu") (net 2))
 (segment (start 91.175 60.5) (end 92.525 61.85) (width 0.5) (layer "F.Cu") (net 2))
 (segment (start 86.25 58.25) (end 87.25 58.25) (width 0.5) (layer "F.Cu") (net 2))
 (segment (start 81.975 67.5) (end 81.975 66) (width 0.5) (layer "F.Cu") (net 2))
 (segment (start 96.8 70.8) (end 98.5 70.8) (width 0.5) (layer "F.Cu") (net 2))
 (segment (start 104.8 70.2) (end 104.4 70.2) (width 0.5) (layer "F.Cu") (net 2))
 (segment (start 103.8 70.8) (end 99.65 70.8) (width 0.5) (layer "F.Cu") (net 2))
 (segment (start 87 75) (end 105.28 75) (width 0.5) (layer "F.Cu") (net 2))
 (segment (start 92.5 56) (end 93 56.5) (width 0.5) (layer "F.Cu") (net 2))
 (segment (start 94 65.3) (end 94.1 65.4) (width 0.5) (layer "F.Cu") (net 2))
 (segment (start 104.775 65.75) (end 104.775 67.6) (width 0.5) (layer "F.Cu") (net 2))
 (segment (start 104.4 70.2) (end 103.8 70.8) (width 0.5) (layer "F.Cu") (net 2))
 (via (at 82 71.5) (size 0.8) (drill 0.4) (layers "F.Cu" "B.Cu") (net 2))
 (via (at 86.25 58.25) (size 0.8) (drill 0.4) (layers "F.Cu" "B.Cu") (free yes) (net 2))
 (via (at 86.25 56) (size 0.8) (drill 0.4) (layers "F.Cu" "B.Cu") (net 2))
 (via (at 81.975 69) (size 0.8) (drill 0.4) (layers "F.Cu" "B.Cu") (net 2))
 (segment (start 86.25 56) (end 86.25 58.25) (width 0.5) (layer "B.Cu") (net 2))
 (segment (start 82 69.025) (end 81.975 69) (width 0.5) (layer "B.Cu") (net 2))
 (segment (start 82 71.5) (end 82 69.025) (width 0.5) (layer "B.Cu") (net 2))
 (segment (start 79 61.25) (end 82 61.25) (width 0.5) (layer "F.Cu") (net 3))
 (segment (start 82 61.25) (end 84.35 63.6) (width 0.5) (layer "F.Cu") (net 3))
 (segment (start 83.525 64.5) (end 83.525 62.775) (width 0.5) (layer "F.Cu") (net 3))
 (segment (start 84.35 63.6) (end 88.35 63.6) (width 0.3) (layer "F.Cu") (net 3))
 (segment (start 83.525 62.775) (end 83.375 62.625) (width 0.5) (layer "F.Cu") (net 3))
 (segment (start 83.525 67.5) (end 83.525 66) (width 0.5) (layer "F.Cu") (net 5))
 (segment (start 88.45 65.9) (end 85.5 65.9) (width 0.5) (layer "F.Cu") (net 5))
 (segment (start 83.525 66) (end 85.4 66) (width 0.5) (layer "F.Cu") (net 5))
 (segment (start 85.5 65.9) (end 85.4 66) (width 0.2) (layer "F.Cu") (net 5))
 (segment (start 85.4 64.401649) (end 85.4 66) (width 0.5) (layer "F.Cu") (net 5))
 (segment (start 97 57.25) (end 97 60.25) (width 0.5) (layer "F.Cu") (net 7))
 (segment (start 100.5 61) (end 101.25 61.75) (width 0.5) (layer "F.Cu") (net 7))
 (segment (start 101.25 61.75) (end 101.25 65.1) (width 0.5) (layer "F.Cu") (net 7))
 (segment (start 97 60.25) (end 97.75 61) (width 0.5) (layer "F.Cu") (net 7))
 (segment (start 103.225 61) (end 100.5 61) (width 0.5) (layer "F.Cu") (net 7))
 (segment (start 101.25 65.1) (end 99.75 65.1) (width 0.5) (layer "F.Cu") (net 7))
 (segment (start 97.75 61) (end 100.5 61) (width 0.5) (layer "F.Cu") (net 7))
 (segment (start 95 57.25) (end 95.3 57.55) (width 0.5) (layer "F.Cu") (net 10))
 (segment (start 95 57.5) (end 95.2 57.7) (width 0.5) (layer "F.Cu") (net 10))
 (segment (start 95.3 57.55) (end 95.3 62.7) (width 0.5) (layer "F.Cu") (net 10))
 (segment (start 95 57.25) (end 95 57.75) (width 0.5) (layer "F.Cu") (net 10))
 (segment (start 95 57.25) (end 95 57.5) (width 0.5) (layer "F.Cu") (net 10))
 (segment (start 91 57.25) (end 92.75 59) (width 0.5) (layer "F.Cu") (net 9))
 (segment (start 94.5 59) (end 94.5 62.7) (width 0.5) (layer "F.Cu") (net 9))
 (segment (start 92.75 59) (end 94.5 59) (width 0.5) (layer "F.Cu") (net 9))
 (segment (start 85.95 57.25) (end 85.4 57.8) (width 0.5) (layer "F.Cu") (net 8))
 (segment (start 89 57.25) (end 85.95 57.25) (width 0.5) (layer "F.Cu") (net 8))
 (segment (start 85.4 57.8) (end 85.4 62.751649) (width 0.5) (layer "F.Cu") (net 8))
 (segment (start 104.93 71.5) (end 105.18 71.75) (width 0.5) (layer "F.Cu") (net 6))
 (segment (start 105.13 73.2) (end 105.28 73.35) (width 0.5) (layer "F.Cu") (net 6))
 (segment (start 99.75 71.5) (end 104.93 71.5) (width 0.5) (layer "F.Cu") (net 6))
 (segment (start 105.13 71.675) (end 105.13 73.2) (width 0.5) (layer "F.Cu") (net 6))
 (segment (start 93.7 61.7) (end 93.7 62.7) (width 0.5) (layer "F.Cu") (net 12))
 (segment (start 92.825 60.825) (end 93.7 61.7) (width 0.5) (layer "F.Cu") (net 12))
 (segment (start 92.825 60.5) (end 92.825 60.825) (width 0.2) (layer "F.Cu") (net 12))
 (segment (start 109.75 71.75) (end 106.83 71.75) (width 0.5) (layer "F.Cu") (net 4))
 (segment (start 106.78 71.675) (end 106.78 73.35) (width 0.5) (layer "F.Cu") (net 4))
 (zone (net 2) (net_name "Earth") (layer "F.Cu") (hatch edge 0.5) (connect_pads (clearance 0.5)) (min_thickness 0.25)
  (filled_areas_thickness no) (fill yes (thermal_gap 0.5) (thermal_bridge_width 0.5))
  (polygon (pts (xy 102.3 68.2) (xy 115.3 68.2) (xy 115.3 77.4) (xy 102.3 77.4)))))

